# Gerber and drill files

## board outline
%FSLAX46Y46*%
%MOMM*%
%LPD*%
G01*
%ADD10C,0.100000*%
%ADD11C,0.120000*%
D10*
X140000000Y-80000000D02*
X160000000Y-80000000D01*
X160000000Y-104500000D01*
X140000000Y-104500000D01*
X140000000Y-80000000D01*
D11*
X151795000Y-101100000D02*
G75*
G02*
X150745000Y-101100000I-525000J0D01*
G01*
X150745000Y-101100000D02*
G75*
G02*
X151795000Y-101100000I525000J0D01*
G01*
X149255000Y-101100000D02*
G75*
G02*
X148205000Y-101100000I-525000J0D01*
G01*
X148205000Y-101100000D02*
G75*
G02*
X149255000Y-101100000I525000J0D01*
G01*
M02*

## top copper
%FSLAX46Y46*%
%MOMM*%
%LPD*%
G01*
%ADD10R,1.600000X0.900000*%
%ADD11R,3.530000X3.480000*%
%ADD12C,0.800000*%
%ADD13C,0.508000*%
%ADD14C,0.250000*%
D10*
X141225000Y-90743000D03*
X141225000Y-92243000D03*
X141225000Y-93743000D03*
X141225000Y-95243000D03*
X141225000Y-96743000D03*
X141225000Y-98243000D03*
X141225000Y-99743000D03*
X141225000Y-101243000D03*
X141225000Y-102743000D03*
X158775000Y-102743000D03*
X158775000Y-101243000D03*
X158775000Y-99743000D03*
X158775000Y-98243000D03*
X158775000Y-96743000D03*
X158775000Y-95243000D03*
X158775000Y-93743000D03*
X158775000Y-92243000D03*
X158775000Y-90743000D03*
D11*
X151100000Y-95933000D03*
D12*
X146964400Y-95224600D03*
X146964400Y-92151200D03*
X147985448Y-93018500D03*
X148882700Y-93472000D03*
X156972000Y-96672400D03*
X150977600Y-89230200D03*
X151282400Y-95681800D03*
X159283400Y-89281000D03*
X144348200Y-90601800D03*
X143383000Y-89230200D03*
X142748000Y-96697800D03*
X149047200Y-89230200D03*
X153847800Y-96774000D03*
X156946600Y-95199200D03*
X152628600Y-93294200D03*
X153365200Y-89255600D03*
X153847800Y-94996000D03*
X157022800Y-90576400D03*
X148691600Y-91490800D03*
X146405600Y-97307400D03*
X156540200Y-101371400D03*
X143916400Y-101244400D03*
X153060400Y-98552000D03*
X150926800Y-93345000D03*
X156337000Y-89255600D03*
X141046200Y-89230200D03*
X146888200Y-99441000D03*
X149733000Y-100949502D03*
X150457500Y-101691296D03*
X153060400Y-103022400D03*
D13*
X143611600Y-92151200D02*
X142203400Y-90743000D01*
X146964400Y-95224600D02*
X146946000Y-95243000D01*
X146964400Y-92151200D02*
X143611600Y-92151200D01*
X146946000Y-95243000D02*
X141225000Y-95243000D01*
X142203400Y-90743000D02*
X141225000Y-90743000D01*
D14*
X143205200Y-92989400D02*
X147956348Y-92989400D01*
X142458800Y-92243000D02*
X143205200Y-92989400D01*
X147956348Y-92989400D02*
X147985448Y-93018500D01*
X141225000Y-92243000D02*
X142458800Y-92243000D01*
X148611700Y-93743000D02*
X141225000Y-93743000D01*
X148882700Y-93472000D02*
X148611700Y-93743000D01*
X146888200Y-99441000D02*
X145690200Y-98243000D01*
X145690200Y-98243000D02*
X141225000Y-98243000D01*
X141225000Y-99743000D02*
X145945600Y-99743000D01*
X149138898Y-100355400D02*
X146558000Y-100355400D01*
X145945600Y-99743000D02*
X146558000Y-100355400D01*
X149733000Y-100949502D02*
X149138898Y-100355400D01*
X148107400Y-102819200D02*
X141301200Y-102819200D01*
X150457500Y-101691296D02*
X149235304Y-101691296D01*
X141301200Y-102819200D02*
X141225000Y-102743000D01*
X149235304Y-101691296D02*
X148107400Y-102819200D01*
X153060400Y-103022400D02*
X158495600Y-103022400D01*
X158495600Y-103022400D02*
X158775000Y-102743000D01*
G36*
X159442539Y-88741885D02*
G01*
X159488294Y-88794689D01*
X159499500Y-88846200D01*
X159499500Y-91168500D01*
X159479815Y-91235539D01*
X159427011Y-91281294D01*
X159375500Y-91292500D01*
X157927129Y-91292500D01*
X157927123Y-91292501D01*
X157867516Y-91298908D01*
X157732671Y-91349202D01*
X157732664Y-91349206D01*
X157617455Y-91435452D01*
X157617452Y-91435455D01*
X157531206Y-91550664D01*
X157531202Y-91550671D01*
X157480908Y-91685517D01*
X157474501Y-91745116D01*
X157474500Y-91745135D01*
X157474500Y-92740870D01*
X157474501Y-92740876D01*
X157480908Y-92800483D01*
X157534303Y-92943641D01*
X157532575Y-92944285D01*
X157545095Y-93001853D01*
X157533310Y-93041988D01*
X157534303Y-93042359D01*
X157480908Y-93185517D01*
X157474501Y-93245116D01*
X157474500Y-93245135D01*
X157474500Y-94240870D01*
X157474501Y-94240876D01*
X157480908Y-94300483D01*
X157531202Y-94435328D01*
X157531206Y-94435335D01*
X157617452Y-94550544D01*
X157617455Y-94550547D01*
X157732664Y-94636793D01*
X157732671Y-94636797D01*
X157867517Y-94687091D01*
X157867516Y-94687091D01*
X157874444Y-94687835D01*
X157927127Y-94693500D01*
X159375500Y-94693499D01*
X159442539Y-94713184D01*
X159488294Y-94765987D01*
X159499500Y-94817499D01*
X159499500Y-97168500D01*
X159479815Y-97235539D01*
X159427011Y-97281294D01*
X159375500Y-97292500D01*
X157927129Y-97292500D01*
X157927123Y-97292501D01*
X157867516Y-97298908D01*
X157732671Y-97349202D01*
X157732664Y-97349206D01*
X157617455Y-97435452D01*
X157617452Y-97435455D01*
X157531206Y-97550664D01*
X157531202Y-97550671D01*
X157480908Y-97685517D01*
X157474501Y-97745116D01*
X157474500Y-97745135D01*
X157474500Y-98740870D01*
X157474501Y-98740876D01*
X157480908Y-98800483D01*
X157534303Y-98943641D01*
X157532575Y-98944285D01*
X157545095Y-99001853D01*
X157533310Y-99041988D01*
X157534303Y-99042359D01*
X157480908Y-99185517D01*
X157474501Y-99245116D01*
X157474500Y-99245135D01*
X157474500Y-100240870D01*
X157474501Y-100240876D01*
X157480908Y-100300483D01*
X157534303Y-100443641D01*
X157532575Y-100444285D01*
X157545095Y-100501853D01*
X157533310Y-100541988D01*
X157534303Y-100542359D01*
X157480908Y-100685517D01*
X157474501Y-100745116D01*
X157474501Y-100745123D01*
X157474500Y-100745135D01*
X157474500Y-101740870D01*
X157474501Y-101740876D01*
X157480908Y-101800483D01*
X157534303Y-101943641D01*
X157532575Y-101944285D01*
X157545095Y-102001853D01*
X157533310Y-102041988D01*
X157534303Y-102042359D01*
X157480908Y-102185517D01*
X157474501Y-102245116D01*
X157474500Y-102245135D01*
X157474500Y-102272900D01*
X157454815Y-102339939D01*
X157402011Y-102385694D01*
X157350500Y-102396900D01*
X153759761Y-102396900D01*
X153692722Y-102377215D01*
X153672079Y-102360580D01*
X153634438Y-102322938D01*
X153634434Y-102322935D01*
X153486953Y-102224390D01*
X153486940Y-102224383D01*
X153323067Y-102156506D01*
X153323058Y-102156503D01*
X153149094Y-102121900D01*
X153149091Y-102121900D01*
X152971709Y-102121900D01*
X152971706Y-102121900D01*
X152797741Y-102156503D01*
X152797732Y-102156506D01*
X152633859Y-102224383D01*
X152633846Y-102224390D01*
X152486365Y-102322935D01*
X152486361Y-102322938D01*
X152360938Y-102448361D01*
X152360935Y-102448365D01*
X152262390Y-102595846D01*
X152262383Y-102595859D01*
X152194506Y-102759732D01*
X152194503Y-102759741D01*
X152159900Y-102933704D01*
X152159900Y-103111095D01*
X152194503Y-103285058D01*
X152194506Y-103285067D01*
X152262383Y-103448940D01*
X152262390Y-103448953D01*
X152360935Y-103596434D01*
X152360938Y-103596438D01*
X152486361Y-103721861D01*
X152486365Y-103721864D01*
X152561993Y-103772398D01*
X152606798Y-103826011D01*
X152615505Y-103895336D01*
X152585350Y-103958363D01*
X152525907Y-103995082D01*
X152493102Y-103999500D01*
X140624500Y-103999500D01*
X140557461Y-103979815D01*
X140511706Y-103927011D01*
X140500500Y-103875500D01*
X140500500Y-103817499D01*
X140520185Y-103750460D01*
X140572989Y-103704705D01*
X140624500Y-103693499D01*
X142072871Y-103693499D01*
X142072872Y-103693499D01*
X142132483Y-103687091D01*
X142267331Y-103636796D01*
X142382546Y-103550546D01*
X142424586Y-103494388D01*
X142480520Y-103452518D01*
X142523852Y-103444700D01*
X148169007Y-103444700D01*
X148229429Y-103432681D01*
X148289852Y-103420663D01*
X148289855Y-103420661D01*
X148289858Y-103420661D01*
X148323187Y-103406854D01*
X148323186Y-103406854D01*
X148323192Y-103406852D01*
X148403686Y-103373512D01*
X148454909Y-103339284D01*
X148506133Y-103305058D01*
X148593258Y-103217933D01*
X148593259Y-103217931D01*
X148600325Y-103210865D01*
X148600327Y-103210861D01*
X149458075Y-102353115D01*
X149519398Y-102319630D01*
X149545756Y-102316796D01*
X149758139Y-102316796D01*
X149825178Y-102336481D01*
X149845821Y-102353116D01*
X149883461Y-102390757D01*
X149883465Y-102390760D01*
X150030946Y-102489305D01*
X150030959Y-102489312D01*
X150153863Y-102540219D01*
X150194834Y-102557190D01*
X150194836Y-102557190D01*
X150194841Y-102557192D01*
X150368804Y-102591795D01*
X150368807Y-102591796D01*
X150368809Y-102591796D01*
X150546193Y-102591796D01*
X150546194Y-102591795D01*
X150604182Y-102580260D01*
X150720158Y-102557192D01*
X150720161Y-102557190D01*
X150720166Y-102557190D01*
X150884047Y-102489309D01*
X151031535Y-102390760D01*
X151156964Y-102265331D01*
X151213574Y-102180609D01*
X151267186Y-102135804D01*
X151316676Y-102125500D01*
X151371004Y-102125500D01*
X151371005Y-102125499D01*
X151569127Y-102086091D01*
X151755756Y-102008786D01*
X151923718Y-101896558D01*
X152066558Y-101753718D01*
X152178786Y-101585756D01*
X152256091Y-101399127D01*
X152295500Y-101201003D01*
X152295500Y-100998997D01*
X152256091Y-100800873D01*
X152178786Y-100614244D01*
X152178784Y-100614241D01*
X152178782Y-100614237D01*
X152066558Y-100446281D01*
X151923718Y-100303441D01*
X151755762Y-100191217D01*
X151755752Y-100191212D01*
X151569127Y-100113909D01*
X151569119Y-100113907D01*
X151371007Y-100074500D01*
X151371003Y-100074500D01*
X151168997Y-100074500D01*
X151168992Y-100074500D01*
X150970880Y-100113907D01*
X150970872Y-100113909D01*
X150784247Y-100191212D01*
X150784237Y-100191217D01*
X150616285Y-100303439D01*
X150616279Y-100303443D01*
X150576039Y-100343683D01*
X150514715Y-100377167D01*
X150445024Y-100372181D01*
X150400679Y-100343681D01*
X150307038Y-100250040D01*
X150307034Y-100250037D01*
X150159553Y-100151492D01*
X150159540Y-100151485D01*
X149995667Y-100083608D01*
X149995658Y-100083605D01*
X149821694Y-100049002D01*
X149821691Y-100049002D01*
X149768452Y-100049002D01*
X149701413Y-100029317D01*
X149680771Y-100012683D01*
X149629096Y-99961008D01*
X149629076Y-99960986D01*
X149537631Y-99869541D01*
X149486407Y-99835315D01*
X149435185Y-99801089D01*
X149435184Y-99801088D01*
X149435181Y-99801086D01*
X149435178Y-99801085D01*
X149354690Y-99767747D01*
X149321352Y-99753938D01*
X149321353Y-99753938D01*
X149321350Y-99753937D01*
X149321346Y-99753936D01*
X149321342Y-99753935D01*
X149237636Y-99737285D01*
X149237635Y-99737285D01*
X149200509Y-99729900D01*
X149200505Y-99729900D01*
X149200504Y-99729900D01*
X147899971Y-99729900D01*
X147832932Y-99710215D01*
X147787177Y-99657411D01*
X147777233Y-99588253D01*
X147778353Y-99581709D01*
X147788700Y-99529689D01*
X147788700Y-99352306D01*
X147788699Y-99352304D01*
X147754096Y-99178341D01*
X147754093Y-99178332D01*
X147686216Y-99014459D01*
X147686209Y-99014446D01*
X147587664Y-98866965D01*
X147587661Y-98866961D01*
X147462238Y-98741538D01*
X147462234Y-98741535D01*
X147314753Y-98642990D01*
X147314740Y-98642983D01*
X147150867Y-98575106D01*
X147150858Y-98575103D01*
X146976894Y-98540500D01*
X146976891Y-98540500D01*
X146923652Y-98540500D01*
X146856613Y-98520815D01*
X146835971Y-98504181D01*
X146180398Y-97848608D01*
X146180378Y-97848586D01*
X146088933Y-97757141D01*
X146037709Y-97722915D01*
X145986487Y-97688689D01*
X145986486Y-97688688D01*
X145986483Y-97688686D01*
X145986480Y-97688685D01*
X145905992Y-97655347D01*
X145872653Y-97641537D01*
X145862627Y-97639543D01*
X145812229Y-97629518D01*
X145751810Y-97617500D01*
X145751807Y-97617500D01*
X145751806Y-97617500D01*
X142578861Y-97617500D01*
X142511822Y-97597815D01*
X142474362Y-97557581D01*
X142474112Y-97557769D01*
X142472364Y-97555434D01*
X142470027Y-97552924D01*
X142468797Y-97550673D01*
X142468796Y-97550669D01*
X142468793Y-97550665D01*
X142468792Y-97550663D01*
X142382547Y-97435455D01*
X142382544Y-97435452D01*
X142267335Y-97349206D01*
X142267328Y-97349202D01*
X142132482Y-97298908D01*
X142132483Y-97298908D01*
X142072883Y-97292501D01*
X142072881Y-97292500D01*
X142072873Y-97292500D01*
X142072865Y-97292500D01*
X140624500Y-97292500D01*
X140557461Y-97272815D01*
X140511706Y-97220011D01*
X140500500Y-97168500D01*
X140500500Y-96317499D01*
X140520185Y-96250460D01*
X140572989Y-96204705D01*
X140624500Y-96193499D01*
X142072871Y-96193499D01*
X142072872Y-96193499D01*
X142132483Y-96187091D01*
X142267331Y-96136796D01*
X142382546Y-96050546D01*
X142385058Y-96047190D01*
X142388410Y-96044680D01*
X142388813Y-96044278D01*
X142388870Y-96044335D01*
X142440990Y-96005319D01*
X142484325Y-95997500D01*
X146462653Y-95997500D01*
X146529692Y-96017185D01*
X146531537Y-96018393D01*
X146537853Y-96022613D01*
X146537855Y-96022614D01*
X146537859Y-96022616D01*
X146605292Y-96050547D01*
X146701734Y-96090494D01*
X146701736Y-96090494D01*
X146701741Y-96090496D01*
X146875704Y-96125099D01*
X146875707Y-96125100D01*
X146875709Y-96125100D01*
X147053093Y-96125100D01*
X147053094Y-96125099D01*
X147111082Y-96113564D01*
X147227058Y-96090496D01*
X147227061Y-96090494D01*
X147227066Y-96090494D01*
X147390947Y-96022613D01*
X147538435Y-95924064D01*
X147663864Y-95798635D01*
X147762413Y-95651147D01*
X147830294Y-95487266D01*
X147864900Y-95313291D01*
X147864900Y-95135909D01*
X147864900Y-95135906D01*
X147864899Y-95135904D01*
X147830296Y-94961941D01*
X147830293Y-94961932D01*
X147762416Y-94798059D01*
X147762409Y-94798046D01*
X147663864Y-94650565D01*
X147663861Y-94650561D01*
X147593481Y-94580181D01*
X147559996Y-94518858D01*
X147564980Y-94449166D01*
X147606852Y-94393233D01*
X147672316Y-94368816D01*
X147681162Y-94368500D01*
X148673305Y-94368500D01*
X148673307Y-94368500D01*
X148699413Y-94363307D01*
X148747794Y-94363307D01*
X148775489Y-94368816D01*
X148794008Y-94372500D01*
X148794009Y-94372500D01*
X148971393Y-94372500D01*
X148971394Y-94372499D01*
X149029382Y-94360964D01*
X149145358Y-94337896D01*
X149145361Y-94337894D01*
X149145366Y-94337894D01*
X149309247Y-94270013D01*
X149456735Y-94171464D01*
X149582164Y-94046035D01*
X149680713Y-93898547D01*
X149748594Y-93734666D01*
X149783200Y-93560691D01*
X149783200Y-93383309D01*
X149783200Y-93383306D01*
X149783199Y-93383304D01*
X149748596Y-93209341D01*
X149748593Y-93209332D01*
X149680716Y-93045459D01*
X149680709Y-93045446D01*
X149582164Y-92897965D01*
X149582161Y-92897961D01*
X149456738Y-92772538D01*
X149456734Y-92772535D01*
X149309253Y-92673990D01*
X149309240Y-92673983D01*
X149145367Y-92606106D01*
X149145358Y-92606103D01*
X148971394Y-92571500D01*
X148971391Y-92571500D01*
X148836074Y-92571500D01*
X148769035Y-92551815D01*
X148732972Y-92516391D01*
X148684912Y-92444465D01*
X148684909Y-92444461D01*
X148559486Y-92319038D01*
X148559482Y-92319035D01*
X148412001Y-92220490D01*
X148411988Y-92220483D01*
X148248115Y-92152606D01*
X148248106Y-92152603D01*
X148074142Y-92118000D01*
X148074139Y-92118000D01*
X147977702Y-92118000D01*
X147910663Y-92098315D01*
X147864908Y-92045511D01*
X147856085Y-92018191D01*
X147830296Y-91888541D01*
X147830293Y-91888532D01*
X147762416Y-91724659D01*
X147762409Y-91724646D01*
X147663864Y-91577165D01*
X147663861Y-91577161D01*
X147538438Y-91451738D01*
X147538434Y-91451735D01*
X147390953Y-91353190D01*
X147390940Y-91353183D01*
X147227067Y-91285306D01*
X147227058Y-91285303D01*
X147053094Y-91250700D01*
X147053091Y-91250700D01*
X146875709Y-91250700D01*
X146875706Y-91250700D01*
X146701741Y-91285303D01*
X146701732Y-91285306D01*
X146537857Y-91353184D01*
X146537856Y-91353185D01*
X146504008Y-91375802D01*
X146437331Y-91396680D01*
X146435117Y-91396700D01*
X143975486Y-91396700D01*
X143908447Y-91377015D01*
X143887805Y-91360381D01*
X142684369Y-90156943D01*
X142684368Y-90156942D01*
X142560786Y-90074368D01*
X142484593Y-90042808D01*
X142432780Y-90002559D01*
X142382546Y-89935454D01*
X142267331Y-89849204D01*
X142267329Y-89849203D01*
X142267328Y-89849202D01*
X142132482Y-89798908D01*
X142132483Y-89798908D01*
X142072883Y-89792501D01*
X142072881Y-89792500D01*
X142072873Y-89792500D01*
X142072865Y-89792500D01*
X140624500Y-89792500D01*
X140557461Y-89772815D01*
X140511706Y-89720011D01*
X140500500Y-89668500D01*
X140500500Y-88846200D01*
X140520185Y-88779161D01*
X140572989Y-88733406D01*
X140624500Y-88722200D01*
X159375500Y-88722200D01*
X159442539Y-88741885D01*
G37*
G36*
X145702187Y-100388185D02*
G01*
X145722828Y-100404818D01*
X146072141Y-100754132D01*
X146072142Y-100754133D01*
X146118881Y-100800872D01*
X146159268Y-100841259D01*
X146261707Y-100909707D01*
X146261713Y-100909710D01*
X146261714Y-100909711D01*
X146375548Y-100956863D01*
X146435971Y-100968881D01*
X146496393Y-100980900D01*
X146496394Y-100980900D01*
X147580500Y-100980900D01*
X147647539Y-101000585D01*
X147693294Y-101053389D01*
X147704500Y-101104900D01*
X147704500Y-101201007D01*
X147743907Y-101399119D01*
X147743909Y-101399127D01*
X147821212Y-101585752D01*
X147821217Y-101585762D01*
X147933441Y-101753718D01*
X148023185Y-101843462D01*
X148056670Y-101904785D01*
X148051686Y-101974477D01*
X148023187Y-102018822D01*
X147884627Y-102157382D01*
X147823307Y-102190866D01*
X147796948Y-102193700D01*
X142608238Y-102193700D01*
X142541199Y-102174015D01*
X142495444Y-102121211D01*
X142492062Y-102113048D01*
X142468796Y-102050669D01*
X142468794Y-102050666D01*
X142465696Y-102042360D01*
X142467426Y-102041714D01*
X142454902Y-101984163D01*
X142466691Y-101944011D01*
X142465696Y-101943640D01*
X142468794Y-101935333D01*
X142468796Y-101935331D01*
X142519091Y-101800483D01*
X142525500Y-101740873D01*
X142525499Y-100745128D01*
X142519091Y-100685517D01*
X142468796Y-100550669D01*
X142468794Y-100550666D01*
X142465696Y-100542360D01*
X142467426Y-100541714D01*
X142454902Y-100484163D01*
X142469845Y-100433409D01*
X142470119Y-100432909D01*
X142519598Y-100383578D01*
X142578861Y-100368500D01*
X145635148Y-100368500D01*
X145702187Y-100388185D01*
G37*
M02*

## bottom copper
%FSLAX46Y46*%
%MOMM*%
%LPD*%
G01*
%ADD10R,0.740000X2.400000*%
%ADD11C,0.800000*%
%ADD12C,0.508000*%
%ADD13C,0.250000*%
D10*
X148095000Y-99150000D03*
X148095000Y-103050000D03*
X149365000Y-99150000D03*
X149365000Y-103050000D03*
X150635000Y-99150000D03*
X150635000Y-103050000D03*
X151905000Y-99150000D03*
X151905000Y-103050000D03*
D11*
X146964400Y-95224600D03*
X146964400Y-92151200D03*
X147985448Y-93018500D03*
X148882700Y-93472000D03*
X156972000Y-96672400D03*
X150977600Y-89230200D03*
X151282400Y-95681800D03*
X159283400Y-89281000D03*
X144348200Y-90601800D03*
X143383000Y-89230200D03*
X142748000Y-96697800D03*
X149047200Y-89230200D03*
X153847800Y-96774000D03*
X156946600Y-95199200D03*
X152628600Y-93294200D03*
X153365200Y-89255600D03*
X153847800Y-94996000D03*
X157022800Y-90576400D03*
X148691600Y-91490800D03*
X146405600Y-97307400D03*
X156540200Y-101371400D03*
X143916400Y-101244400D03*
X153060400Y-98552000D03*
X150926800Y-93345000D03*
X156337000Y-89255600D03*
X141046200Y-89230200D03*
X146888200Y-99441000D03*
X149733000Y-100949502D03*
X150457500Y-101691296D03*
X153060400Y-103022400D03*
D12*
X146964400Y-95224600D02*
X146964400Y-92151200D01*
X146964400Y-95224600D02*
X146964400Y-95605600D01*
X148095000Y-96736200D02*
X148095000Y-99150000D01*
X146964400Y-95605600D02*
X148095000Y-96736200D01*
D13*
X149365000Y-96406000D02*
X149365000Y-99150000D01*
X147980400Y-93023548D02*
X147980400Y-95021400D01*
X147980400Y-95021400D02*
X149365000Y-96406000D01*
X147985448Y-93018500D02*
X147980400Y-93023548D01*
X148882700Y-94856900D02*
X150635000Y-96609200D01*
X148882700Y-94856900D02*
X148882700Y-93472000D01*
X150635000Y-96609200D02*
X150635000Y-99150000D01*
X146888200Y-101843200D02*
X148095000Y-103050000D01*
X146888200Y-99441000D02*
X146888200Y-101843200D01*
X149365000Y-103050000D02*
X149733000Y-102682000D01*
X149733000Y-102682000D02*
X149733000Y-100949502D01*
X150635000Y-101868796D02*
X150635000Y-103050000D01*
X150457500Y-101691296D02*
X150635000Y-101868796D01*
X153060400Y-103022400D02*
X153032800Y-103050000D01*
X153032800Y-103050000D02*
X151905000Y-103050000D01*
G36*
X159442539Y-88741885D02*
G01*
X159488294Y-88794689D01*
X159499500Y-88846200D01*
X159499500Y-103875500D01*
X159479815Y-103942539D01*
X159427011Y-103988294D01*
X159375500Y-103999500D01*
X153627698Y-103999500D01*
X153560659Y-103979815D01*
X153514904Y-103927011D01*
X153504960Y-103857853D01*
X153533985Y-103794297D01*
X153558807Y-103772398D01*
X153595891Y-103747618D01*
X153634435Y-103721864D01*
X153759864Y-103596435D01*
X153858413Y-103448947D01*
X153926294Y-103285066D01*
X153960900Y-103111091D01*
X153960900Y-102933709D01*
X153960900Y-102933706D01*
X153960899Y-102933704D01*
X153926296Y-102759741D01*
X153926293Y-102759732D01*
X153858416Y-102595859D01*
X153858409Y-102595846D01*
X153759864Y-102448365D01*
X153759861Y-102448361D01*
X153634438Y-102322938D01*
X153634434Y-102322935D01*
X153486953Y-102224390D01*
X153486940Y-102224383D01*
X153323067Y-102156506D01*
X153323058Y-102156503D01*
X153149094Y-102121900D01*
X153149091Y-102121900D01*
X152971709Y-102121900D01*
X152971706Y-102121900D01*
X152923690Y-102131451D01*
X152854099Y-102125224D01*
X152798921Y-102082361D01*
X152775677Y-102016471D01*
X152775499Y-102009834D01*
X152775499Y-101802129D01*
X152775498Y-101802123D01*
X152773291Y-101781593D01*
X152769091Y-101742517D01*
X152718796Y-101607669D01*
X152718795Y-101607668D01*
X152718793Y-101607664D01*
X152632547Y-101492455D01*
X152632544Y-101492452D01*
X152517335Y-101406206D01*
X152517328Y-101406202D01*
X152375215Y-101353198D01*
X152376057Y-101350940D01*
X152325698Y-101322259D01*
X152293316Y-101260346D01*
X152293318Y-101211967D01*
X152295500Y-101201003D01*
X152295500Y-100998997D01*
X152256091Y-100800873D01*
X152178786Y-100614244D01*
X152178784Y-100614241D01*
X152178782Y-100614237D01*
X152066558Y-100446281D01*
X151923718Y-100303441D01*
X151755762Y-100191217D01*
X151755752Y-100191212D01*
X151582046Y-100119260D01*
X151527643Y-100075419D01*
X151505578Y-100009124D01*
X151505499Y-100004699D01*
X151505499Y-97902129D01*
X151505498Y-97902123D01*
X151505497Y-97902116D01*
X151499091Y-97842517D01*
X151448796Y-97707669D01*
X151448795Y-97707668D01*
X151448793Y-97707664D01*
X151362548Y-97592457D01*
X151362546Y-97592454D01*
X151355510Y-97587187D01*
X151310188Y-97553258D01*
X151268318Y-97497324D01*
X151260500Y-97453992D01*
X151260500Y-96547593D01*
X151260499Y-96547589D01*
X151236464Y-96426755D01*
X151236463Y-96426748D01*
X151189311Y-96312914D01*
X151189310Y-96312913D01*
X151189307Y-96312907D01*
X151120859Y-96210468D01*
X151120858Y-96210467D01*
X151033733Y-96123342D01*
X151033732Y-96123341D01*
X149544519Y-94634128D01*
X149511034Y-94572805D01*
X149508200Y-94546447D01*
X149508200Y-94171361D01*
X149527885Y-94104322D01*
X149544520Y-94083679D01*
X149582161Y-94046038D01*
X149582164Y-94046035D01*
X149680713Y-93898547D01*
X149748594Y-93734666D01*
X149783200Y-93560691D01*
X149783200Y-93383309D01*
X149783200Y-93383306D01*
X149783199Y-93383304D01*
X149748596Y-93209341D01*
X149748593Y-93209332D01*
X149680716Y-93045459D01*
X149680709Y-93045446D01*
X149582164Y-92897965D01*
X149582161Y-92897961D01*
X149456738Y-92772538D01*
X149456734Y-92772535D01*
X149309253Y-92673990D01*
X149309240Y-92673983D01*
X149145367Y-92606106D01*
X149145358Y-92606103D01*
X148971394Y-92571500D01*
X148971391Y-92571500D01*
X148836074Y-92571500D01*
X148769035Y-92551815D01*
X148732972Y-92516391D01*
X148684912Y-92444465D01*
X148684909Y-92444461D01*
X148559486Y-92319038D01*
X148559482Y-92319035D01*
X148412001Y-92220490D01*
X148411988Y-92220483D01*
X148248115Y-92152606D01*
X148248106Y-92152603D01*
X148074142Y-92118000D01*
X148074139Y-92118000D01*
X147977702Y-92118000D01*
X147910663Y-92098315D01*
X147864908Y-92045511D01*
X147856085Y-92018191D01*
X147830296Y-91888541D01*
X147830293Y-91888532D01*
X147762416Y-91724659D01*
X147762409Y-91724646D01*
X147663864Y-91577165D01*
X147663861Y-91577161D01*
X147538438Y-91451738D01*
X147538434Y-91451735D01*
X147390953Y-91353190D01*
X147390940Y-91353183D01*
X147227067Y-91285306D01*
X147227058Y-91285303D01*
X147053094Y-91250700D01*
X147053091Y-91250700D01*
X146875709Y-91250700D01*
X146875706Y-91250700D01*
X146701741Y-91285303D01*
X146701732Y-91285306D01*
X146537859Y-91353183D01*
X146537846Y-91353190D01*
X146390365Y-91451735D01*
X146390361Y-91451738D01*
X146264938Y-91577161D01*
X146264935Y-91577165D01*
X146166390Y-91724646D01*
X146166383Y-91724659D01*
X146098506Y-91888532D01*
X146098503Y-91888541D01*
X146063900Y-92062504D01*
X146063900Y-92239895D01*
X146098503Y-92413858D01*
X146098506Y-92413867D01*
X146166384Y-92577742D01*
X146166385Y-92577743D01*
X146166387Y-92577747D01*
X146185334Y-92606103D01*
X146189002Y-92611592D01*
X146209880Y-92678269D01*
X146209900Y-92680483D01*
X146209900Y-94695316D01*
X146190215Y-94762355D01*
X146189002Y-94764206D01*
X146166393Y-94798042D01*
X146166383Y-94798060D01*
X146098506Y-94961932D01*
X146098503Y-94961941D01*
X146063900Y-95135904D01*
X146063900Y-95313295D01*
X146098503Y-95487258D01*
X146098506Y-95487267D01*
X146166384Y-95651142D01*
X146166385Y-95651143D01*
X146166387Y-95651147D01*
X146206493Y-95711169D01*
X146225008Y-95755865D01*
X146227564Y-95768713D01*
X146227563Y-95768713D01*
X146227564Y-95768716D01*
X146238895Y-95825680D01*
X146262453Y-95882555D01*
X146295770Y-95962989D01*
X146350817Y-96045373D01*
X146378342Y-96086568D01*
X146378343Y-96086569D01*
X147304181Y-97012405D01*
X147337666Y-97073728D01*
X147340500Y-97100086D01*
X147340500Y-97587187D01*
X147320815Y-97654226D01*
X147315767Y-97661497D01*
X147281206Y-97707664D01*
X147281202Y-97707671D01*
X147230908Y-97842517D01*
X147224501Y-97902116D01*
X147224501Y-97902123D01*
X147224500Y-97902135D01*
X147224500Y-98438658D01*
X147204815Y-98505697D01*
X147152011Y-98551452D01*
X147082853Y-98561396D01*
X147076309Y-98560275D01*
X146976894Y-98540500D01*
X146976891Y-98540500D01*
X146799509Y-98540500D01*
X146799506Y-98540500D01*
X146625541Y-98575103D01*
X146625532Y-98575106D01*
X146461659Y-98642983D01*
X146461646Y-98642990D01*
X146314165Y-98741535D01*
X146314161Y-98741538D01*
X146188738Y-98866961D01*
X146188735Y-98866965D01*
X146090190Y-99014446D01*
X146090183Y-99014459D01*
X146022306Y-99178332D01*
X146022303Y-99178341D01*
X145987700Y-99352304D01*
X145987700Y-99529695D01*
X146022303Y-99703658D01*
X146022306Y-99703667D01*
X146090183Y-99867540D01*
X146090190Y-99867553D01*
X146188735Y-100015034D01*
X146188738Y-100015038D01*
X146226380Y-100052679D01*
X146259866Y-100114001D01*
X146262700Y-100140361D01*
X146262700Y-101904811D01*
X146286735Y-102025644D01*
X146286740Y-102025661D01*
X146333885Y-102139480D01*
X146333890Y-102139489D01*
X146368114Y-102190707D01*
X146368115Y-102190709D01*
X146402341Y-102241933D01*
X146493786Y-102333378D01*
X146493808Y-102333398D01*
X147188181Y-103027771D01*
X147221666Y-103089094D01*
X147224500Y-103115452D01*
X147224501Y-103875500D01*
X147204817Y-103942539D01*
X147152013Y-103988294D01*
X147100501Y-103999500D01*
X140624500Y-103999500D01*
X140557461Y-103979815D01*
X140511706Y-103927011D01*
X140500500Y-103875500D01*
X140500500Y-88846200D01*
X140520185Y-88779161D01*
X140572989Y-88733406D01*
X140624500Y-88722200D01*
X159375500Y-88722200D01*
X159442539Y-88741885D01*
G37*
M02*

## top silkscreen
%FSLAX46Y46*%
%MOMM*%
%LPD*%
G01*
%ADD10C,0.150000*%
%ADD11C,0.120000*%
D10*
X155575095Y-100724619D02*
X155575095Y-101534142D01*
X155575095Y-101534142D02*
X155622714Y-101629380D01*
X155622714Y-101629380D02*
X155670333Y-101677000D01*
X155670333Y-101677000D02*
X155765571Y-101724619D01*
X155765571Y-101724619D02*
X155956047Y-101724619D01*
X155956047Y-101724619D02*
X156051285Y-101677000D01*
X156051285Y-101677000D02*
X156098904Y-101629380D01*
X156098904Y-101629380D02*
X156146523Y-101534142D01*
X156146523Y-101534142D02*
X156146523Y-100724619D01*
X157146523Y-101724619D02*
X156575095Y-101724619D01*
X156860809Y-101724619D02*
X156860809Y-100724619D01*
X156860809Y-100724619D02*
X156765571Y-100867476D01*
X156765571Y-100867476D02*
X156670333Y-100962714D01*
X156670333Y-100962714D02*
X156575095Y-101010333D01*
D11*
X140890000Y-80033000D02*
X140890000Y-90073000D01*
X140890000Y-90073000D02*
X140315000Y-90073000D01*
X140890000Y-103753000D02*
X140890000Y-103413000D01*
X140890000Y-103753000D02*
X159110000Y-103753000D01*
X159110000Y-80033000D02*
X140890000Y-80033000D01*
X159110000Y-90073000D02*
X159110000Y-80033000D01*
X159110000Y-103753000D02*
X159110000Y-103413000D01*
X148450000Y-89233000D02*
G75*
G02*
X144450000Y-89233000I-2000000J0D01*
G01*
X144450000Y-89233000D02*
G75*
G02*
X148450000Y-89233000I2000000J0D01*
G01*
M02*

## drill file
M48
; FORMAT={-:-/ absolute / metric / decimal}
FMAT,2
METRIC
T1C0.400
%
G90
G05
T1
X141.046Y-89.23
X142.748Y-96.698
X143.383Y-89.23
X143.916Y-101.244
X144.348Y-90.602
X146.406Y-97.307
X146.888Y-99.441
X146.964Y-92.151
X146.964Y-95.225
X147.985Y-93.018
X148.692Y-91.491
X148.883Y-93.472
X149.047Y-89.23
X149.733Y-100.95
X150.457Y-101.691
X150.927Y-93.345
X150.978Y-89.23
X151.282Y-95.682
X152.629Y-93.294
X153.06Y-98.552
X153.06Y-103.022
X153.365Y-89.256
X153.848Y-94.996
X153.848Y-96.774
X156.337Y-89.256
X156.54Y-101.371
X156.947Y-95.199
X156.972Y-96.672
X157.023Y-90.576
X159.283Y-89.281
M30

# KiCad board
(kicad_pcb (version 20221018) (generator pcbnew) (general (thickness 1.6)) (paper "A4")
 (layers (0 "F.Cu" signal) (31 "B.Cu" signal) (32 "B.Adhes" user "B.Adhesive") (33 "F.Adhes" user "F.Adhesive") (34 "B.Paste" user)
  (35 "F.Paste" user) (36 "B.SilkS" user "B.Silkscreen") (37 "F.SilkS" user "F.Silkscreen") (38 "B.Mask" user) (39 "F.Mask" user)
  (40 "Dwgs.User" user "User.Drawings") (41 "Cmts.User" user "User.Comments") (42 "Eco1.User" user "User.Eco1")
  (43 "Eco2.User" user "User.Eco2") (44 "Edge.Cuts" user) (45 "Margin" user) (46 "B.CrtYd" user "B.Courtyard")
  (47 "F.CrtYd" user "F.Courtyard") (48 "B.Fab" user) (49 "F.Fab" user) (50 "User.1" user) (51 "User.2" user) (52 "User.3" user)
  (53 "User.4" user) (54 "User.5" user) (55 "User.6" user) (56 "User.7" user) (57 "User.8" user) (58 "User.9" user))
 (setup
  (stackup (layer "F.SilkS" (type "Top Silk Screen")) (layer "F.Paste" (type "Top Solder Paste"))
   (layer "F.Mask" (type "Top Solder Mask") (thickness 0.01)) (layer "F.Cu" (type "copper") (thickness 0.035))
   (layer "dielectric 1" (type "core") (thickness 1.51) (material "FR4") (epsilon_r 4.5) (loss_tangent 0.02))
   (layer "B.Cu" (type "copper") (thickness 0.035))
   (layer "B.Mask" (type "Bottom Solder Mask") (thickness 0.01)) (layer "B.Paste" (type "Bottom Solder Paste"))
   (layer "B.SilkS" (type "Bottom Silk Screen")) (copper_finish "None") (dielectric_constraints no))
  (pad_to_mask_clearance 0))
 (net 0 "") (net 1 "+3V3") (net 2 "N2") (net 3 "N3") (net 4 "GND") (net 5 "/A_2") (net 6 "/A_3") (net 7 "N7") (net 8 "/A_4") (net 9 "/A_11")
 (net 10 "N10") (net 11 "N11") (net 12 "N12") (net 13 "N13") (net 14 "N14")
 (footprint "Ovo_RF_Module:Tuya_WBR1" (layer "F.Cu") (at 150 96.743)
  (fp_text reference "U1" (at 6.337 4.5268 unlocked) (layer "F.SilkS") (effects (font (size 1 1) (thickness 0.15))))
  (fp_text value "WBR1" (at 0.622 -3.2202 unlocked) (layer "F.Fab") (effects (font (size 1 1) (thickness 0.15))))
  (fp_line (start -9.11 -16.71) (end -9.11 -6.67) (stroke (width 0.12) (type solid)) (layer "F.SilkS"))
  (fp_line (start -9.11 -6.67) (end -9.685 -6.67) (stroke (width 0.12) (type solid)) (layer "F.SilkS"))
  (fp_line (start -9.11 7.01) (end -9.11 6.67) (stroke (width 0.12) (type solid)) (layer "F.SilkS"))
  (fp_line (start -9.11 7.01) (end 9.11 7.01) (stroke (width 0.12) (type solid)) (layer "F.SilkS"))
  (fp_line (start 9.11 -16.71) (end -9.11 -16.71) (stroke (width 0.12) (type solid)) (layer "F.SilkS"))
  (fp_line (start 9.11 -6.67) (end 9.11 -16.71) (stroke (width 0.12) (type solid)) (layer "F.SilkS"))
  (fp_line (start 9.11 7.01) (end 9.11 6.67) (stroke (width 0.12) (type solid)) (layer "F.SilkS"))
  (fp_circle (center -3.55 -7.51) (end -1.55 -7.51) (stroke (width 0.12) (type solid)) (fill none) (layer "F.SilkS"))
  (pad "1" smd rect (at -8.775 -6) (size 1.6 0.9) (layers "F.Cu" "F.Paste" "F.Mask") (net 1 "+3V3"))
  (pad "2" smd rect (at -8.775 -4.5) (size 1.6 0.9) (layers "F.Cu" "F.Paste" "F.Mask") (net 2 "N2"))
  (pad "3" smd rect (at -8.775 -3) (size 1.6 0.9) (layers "F.Cu" "F.Paste" "F.Mask") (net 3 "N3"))
  (pad "4" smd rect (at -8.775 -1.5) (size 1.6 0.9) (layers "F.Cu" "F.Paste" "F.Mask") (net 1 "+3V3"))
  (pad "5" smd rect (at -8.775 0) (size 1.6 0.9) (layers "F.Cu" "F.Paste" "F.Mask") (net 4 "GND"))
  (pad "6" smd rect (at -8.775 1.5) (size 1.6 0.9) (layers "F.Cu" "F.Paste" "F.Mask") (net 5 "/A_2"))
  (pad "7" smd rect (at -8.775 3) (size 1.6 0.9) (layers "F.Cu" "F.Paste" "F.Mask") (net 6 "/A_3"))
  (pad "8" smd rect (at -8.775 4.5) (size 1.6 0.9) (layers "F.Cu" "F.Paste" "F.Mask") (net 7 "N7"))
  (pad "9" smd rect (at -8.775 6) (size 1.6 0.9) (layers "F.Cu" "F.Paste" "F.Mask") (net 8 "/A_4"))
  (pad "10" smd rect (at 8.775 6) (size 1.6 0.9) (layers "F.Cu" "F.Paste" "F.Mask") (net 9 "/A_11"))
  (pad "11" smd rect (at 8.775 4.5) (size 1.6 0.9) (layers "F.Cu" "F.Paste" "F.Mask") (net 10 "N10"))
  (pad "12" smd rect (at 8.775 3) (size 1.6 0.9) (layers "F.Cu" "F.Paste" "F.Mask") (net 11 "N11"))
  (pad "13" smd rect (at 8.775 1.5) (size 1.6 0.9) (layers "F.Cu" "F.Paste" "F.Mask") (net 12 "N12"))
  (pad "14" smd rect (at 8.775 0) (size 1.6 0.9) (layers "F.Cu" "F.Paste" "F.Mask") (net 4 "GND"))
  (pad "15" smd rect (at 8.775 -1.5) (size 1.6 0.9) (layers "F.Cu" "F.Paste" "F.Mask") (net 4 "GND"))
  (pad "16" smd rect (at 8.775 -3) (size 1.6 0.9) (layers "F.Cu" "F.Paste" "F.Mask") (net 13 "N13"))
  (pad "17" smd rect (at 8.775 -4.5) (size 1.6 0.9) (layers "F.Cu" "F.Paste" "F.Mask") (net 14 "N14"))
  (pad "18" smd rect (at 8.775 -6) (size 1.6 0.9) (layers "F.Cu" "F.Paste" "F.Mask") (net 4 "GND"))
  (pad "19" smd rect (at 1.1 -0.81) (size 3.53 3.48) (layers "F.Cu" "F.Paste" "F.Mask") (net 4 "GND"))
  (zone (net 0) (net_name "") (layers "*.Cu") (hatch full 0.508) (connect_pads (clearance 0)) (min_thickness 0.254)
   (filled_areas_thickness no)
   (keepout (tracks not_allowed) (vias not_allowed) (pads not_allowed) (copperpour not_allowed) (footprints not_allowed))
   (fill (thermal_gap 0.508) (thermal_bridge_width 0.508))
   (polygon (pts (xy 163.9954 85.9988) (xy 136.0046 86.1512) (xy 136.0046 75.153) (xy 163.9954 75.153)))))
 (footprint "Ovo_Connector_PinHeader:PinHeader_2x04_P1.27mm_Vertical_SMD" (layer "B.Cu") (at 150 101.1 -90)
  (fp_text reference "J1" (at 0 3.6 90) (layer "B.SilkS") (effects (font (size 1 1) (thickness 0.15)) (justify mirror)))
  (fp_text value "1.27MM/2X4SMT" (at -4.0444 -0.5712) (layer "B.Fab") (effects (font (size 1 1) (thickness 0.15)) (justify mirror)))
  (fp_circle (center 0 -1.27) (end 0.525 -1.27) (stroke (width 0.12) (type default)) (fill none) (layer "Edge.Cuts"))
  (fp_circle (center 0 1.27) (end 0.525 1.27) (stroke (width 0.12) (type default)) (fill none) (layer "Edge.Cuts"))
  (pad "1" smd rect (at -1.95 1.905 270) (size 2.4 0.74) (layers "B.Cu" "B.Paste" "B.Mask") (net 1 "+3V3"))
  (pad "2" smd rect (at 1.95 1.905 270) (size 2.4 0.74) (layers "B.Cu" "B.Paste" "B.Mask") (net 5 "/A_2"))
  (pad "3" smd rect (at -1.95 0.635 270) (size 2.4 0.74) (layers "B.Cu" "B.Paste" "B.Mask") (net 2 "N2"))
  (pad "4" smd rect (at 1.95 0.635 270) (size 2.4 0.74) (layers "B.Cu" "B.Paste" "B.Mask") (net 6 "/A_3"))
  (pad "5" smd rect (at -1.95 -0.635 270) (size 2.4 0.74) (layers "B.Cu" "B.Paste" "B.Mask") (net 3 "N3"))
  (pad "6" smd rect (at 1.95 -0.635 270) (size 2.4 0.74) (layers "B.Cu" "B.Paste" "B.Mask") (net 8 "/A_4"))
  (pad "7" smd rect (at -1.95 -1.905 270) (size 2.4 0.74) (layers "B.Cu" "B.Paste" "B.Mask") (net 4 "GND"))
  (pad "8" smd rect (at 1.95 -1.905 270) (size 2.4 0.74) (layers "B.Cu" "B.Paste" "B.Mask") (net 9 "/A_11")))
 (gr_rect (start 140 80) (end 160 104.5) (stroke (width 0.1) (type default)) (fill none) (layer "Edge.Cuts"))
 (segment (start 143.6116 92.1512) (end 142.2034 90.743) (width 0.508) (layer "F.Cu") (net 1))
 (segment (start 146.9644 95.2246) (end 146.946 95.243) (width 0.508) (layer "F.Cu") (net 1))
 (segment (start 146.9644 92.1512) (end 143.6116 92.1512) (width 0.508) (layer "F.Cu") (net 1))
 (segment (start 146.946 95.243) (end 141.225 95.243) (width 0.508) (layer "F.Cu") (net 1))
 (segment (start 142.2034 90.743) (end 141.225 90.743) (width 0.508) (layer "F.Cu") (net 1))
 (via (at 146.9644 95.2246) (size 0.8) (drill 0.4) (layers "F.Cu" "B.Cu") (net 1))
 (via (at 146.9644 92.1512) (size 0.8) (drill 0.4) (layers "F.Cu" "B.Cu") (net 1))
 (segment (start 146.9644 95.2246) (end 146.9644 92.1512) (width 0.508) (layer "B.Cu") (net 1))
 (segment (start 146.9644 95.2246) (end 146.9644 95.6056) (width 0.508) (layer "B.Cu") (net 1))
 (segment (start 148.095 96.7362) (end 148.095 99.15) (width 0.508) (layer "B.Cu") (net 1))
 (segment (start 146.9644 95.6056) (end 148.095 96.7362) (width 0.508) (layer "B.Cu") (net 1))
 (segment (start 143.2052 92.9894) (end 147.956348 92.9894) (width 0.25) (layer "F.Cu") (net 2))
 (segment (start 142.4588 92.243) (end 143.2052 92.9894) (width 0.25) (layer "F.Cu") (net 2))
 (segment (start 147.956348 92.9894) (end 147.985448 93.0185) (width 0.25) (layer "F.Cu") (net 2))
 (segment (start 141.225 92.243) (end 142.4588 92.243) (width 0.25) (layer "F.Cu") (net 2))
 (via (at 147.985448 93.0185) (size 0.8) (drill 0.4) (layers "F.Cu" "B.Cu") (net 2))
 (segment (start 149.365 96.406) (end 149.365 99.15) (width 0.25) (layer "B.Cu") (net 2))
 (segment (start 147.9804 93.023548) (end 147.9804 95.0214) (width 0.25) (layer "B.Cu") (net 2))
 (segment (start 147.9804 95.0214) (end 149.365 96.406) (width 0.25) (layer "B.Cu") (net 2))
 (segment (start 147.985448 93.0185) (end 147.9804 93.023548) (width 0.25) (layer "B.Cu") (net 2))
 (segment (start 148.6117 93.743) (end 141.225 93.743) (width 0.25) (layer "F.Cu") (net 3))
 (segment (start 148.8827 93.472) (end 148.6117 93.743) (width 0.25) (layer "F.Cu") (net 3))
 (via (at 148.8827 93.472) (size 0.8) (drill 0.4) (layers "F.Cu" "B.Cu") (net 3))
 (segment (start 148.8827 94.8569) (end 150.635 96.6092) (width 0.25) (layer "B.Cu") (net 3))
 (segment (start 148.8827 94.8569) (end 148.8827 93.472) (width 0.25) (layer "B.Cu") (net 3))
 (segment (start 150.635 96.6092) (end 150.635 99.15) (width 0.25) (layer "B.Cu") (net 3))
 (via (at 156.972 96.6724) (size 0.8) (drill 0.4) (layers "F.Cu" "B.Cu") (free) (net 4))
 (via (at 150.9776 89.2302) (size 0.8) (drill 0.4) (layers "F.Cu" "B.Cu") (free) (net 4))
 (via (at 151.2824 95.6818) (size 0.8) (drill 0.4) (layers "F.Cu" "B.Cu") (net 4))
 (via (at 159.2834 89.281) (size 0.8) (drill 0.4) (layers "F.Cu" "B.Cu") (free) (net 4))
 (via (at 144.3482 90.6018) (size 0.8) (drill 0.4) (layers "F.Cu" "B.Cu") (free) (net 4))
 (via (at 143.383 89.2302) (size 0.8) (drill 0.4) (layers "F.Cu" "B.Cu") (free) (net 4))
 (via (at 142.748 96.6978) (size 0.8) (drill 0.4) (layers "F.Cu" "B.Cu") (free) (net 4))
 (via (at 149.0472 89.2302) (size 0.8) (drill 0.4) (layers "F.Cu" "B.Cu") (free) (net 4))
 (via (at 153.8478 96.774) (size 0.8) (drill 0.4) (layers "F.Cu" "B.Cu") (free) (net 4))
 (via (at 156.9466 95.1992) (size 0.8) (drill 0.4) (layers "F.Cu" "B.Cu") (free) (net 4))
 (via (at 152.6286 93.2942) (size 0.8) (drill 0.4) (layers "F.Cu" "B.Cu") (free) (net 4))
 (via (at 153.3652 89.2556) (size 0.8) (drill 0.4) (layers "F.Cu" "B.Cu") (free) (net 4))
 (via (at 153.8478 94.996) (size 0.8) (drill 0.4) (layers "F.Cu" "B.Cu") (free) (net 4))
 (via (at 157.0228 90.5764) (size 0.8) (drill 0.4) (layers "F.Cu" "B.Cu") (free) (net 4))
 (via (at 148.6916 91.4908) (size 0.8) (drill 0.4) (layers "F.Cu" "B.Cu") (free) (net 4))
 (via (at 146.4056 97.3074) (size 0.8) (drill 0.4) (layers "F.Cu" "B.Cu") (free) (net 4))
 (via (at 156.5402 101.3714) (size 0.8) (drill 0.4) (layers "F.Cu" "B.Cu") (free) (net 4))
 (via (at 143.9164 101.2444) (size 0.8) (drill 0.4) (layers "F.Cu" "B.Cu") (free) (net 4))
 (via (at 153.0604 98.552) (size 0.8) (drill 0.4) (layers "F.Cu" "B.Cu") (free) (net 4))
 (via (at 150.9268 93.345) (size 0.8) (drill 0.4) (layers "F.Cu" "B.Cu") (free) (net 4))
 (via (at 156.337 89.2556) (size 0.8) (drill 0.4) (layers "F.Cu" "B.Cu") (free) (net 4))
 (via (at 141.0462 89.2302) (size 0.8) (drill 0.4) (layers "F.Cu" "B.Cu") (free) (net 4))
 (segment (start 146.8882 99.441) (end 145.6902 98.243) (width 0.25) (layer "F.Cu") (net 5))
 (segment (start 145.6902 98.243) (end 141.225 98.243) (width 0.25) (layer "F.Cu") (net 5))
 (via (at 146.8882 99.441) (size 0.8) (drill 0.4) (layers "F.Cu" "B.Cu") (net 5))
 (segment (start 146.8882 101.8432) (end 148.095 103.05) (width 0.25) (layer "B.Cu") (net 5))
 (segment (start 146.8882 99.441) (end 146.8882 101.8432) (width 0.25) (layer "B.Cu") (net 5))
 (segment (start 141.225 99.743) (end 145.9456 99.743) (width 0.25) (layer "F.Cu") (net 6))
 (segment (start 149.138898 100.3554) (end 146.558 100.3554) (width 0.25) (layer "F.Cu") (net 6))
 (segment (start 145.9456 99.743) (end 146.558 100.3554) (width 0.25) (layer "F.Cu") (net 6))
 (segment (start 149.733 100.949502) (end 149.138898 100.3554) (width 0.25) (layer "F.Cu") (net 6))
 (via (at 149.733 100.949502) (size 0.8) (drill 0.4) (layers "F.Cu" "B.Cu") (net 6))
 (segment (start 149.365 103.05) (end 149.733 102.682) (width 0.25) (layer "B.Cu") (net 6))
 (segment (start 149.733 102.682) (end 149.733 100.949502) (width 0.25) (layer "B.Cu") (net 6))
 (segment (start 148.1074 102.8192) (end 141.3012 102.8192) (width 0.25) (layer "F.Cu") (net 8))
 (segment (start 150.4575 101.691296) (end 149.235304 101.691296) (width 0.25) (layer "F.Cu") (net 8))
 (segment (start 141.3012 102.8192) (end 141.225 102.743) (width 0.25) (layer "F.Cu") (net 8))
 (segment (start 149.235304 101.691296) (end 148.1074 102.8192) (width 0.25) (layer "F.Cu") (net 8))
 (via (at 150.4575 101.691296) (size 0.8) (drill 0.4) (layers "F.Cu" "B.Cu") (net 8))
 (segment (start 150.635 101.868796) (end 150.635 103.05) (width 0.25) (layer "B.Cu") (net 8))
 (segment (start 150.4575 101.691296) (end 150.635 101.868796) (width 0.25) (layer "B.Cu") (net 8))
 (segment (start 153.0604 103.0224) (end 158.4956 103.0224) (width 0.25) (layer "F.Cu") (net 9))
 (segment (start 158.4956 103.0224) (end 158.775 102.743) (width 0.25) (layer "F.Cu") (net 9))
 (via (at 153.0604 103.0224) (size 0.8) (drill 0.4) (layers "F.Cu" "B.Cu") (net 9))
 (segment (start 153.0604 103.0224) (end 153.0328 103.05) (width 0.25) (layer "B.Cu") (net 9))
 (segment (start 153.0328 103.05) (end 151.905 103.05) (width 0.25) (layer "B.Cu") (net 9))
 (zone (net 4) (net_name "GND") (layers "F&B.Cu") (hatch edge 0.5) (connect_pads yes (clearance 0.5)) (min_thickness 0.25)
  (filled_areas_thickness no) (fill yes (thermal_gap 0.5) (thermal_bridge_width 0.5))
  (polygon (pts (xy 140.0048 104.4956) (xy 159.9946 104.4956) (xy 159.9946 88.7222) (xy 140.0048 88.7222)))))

